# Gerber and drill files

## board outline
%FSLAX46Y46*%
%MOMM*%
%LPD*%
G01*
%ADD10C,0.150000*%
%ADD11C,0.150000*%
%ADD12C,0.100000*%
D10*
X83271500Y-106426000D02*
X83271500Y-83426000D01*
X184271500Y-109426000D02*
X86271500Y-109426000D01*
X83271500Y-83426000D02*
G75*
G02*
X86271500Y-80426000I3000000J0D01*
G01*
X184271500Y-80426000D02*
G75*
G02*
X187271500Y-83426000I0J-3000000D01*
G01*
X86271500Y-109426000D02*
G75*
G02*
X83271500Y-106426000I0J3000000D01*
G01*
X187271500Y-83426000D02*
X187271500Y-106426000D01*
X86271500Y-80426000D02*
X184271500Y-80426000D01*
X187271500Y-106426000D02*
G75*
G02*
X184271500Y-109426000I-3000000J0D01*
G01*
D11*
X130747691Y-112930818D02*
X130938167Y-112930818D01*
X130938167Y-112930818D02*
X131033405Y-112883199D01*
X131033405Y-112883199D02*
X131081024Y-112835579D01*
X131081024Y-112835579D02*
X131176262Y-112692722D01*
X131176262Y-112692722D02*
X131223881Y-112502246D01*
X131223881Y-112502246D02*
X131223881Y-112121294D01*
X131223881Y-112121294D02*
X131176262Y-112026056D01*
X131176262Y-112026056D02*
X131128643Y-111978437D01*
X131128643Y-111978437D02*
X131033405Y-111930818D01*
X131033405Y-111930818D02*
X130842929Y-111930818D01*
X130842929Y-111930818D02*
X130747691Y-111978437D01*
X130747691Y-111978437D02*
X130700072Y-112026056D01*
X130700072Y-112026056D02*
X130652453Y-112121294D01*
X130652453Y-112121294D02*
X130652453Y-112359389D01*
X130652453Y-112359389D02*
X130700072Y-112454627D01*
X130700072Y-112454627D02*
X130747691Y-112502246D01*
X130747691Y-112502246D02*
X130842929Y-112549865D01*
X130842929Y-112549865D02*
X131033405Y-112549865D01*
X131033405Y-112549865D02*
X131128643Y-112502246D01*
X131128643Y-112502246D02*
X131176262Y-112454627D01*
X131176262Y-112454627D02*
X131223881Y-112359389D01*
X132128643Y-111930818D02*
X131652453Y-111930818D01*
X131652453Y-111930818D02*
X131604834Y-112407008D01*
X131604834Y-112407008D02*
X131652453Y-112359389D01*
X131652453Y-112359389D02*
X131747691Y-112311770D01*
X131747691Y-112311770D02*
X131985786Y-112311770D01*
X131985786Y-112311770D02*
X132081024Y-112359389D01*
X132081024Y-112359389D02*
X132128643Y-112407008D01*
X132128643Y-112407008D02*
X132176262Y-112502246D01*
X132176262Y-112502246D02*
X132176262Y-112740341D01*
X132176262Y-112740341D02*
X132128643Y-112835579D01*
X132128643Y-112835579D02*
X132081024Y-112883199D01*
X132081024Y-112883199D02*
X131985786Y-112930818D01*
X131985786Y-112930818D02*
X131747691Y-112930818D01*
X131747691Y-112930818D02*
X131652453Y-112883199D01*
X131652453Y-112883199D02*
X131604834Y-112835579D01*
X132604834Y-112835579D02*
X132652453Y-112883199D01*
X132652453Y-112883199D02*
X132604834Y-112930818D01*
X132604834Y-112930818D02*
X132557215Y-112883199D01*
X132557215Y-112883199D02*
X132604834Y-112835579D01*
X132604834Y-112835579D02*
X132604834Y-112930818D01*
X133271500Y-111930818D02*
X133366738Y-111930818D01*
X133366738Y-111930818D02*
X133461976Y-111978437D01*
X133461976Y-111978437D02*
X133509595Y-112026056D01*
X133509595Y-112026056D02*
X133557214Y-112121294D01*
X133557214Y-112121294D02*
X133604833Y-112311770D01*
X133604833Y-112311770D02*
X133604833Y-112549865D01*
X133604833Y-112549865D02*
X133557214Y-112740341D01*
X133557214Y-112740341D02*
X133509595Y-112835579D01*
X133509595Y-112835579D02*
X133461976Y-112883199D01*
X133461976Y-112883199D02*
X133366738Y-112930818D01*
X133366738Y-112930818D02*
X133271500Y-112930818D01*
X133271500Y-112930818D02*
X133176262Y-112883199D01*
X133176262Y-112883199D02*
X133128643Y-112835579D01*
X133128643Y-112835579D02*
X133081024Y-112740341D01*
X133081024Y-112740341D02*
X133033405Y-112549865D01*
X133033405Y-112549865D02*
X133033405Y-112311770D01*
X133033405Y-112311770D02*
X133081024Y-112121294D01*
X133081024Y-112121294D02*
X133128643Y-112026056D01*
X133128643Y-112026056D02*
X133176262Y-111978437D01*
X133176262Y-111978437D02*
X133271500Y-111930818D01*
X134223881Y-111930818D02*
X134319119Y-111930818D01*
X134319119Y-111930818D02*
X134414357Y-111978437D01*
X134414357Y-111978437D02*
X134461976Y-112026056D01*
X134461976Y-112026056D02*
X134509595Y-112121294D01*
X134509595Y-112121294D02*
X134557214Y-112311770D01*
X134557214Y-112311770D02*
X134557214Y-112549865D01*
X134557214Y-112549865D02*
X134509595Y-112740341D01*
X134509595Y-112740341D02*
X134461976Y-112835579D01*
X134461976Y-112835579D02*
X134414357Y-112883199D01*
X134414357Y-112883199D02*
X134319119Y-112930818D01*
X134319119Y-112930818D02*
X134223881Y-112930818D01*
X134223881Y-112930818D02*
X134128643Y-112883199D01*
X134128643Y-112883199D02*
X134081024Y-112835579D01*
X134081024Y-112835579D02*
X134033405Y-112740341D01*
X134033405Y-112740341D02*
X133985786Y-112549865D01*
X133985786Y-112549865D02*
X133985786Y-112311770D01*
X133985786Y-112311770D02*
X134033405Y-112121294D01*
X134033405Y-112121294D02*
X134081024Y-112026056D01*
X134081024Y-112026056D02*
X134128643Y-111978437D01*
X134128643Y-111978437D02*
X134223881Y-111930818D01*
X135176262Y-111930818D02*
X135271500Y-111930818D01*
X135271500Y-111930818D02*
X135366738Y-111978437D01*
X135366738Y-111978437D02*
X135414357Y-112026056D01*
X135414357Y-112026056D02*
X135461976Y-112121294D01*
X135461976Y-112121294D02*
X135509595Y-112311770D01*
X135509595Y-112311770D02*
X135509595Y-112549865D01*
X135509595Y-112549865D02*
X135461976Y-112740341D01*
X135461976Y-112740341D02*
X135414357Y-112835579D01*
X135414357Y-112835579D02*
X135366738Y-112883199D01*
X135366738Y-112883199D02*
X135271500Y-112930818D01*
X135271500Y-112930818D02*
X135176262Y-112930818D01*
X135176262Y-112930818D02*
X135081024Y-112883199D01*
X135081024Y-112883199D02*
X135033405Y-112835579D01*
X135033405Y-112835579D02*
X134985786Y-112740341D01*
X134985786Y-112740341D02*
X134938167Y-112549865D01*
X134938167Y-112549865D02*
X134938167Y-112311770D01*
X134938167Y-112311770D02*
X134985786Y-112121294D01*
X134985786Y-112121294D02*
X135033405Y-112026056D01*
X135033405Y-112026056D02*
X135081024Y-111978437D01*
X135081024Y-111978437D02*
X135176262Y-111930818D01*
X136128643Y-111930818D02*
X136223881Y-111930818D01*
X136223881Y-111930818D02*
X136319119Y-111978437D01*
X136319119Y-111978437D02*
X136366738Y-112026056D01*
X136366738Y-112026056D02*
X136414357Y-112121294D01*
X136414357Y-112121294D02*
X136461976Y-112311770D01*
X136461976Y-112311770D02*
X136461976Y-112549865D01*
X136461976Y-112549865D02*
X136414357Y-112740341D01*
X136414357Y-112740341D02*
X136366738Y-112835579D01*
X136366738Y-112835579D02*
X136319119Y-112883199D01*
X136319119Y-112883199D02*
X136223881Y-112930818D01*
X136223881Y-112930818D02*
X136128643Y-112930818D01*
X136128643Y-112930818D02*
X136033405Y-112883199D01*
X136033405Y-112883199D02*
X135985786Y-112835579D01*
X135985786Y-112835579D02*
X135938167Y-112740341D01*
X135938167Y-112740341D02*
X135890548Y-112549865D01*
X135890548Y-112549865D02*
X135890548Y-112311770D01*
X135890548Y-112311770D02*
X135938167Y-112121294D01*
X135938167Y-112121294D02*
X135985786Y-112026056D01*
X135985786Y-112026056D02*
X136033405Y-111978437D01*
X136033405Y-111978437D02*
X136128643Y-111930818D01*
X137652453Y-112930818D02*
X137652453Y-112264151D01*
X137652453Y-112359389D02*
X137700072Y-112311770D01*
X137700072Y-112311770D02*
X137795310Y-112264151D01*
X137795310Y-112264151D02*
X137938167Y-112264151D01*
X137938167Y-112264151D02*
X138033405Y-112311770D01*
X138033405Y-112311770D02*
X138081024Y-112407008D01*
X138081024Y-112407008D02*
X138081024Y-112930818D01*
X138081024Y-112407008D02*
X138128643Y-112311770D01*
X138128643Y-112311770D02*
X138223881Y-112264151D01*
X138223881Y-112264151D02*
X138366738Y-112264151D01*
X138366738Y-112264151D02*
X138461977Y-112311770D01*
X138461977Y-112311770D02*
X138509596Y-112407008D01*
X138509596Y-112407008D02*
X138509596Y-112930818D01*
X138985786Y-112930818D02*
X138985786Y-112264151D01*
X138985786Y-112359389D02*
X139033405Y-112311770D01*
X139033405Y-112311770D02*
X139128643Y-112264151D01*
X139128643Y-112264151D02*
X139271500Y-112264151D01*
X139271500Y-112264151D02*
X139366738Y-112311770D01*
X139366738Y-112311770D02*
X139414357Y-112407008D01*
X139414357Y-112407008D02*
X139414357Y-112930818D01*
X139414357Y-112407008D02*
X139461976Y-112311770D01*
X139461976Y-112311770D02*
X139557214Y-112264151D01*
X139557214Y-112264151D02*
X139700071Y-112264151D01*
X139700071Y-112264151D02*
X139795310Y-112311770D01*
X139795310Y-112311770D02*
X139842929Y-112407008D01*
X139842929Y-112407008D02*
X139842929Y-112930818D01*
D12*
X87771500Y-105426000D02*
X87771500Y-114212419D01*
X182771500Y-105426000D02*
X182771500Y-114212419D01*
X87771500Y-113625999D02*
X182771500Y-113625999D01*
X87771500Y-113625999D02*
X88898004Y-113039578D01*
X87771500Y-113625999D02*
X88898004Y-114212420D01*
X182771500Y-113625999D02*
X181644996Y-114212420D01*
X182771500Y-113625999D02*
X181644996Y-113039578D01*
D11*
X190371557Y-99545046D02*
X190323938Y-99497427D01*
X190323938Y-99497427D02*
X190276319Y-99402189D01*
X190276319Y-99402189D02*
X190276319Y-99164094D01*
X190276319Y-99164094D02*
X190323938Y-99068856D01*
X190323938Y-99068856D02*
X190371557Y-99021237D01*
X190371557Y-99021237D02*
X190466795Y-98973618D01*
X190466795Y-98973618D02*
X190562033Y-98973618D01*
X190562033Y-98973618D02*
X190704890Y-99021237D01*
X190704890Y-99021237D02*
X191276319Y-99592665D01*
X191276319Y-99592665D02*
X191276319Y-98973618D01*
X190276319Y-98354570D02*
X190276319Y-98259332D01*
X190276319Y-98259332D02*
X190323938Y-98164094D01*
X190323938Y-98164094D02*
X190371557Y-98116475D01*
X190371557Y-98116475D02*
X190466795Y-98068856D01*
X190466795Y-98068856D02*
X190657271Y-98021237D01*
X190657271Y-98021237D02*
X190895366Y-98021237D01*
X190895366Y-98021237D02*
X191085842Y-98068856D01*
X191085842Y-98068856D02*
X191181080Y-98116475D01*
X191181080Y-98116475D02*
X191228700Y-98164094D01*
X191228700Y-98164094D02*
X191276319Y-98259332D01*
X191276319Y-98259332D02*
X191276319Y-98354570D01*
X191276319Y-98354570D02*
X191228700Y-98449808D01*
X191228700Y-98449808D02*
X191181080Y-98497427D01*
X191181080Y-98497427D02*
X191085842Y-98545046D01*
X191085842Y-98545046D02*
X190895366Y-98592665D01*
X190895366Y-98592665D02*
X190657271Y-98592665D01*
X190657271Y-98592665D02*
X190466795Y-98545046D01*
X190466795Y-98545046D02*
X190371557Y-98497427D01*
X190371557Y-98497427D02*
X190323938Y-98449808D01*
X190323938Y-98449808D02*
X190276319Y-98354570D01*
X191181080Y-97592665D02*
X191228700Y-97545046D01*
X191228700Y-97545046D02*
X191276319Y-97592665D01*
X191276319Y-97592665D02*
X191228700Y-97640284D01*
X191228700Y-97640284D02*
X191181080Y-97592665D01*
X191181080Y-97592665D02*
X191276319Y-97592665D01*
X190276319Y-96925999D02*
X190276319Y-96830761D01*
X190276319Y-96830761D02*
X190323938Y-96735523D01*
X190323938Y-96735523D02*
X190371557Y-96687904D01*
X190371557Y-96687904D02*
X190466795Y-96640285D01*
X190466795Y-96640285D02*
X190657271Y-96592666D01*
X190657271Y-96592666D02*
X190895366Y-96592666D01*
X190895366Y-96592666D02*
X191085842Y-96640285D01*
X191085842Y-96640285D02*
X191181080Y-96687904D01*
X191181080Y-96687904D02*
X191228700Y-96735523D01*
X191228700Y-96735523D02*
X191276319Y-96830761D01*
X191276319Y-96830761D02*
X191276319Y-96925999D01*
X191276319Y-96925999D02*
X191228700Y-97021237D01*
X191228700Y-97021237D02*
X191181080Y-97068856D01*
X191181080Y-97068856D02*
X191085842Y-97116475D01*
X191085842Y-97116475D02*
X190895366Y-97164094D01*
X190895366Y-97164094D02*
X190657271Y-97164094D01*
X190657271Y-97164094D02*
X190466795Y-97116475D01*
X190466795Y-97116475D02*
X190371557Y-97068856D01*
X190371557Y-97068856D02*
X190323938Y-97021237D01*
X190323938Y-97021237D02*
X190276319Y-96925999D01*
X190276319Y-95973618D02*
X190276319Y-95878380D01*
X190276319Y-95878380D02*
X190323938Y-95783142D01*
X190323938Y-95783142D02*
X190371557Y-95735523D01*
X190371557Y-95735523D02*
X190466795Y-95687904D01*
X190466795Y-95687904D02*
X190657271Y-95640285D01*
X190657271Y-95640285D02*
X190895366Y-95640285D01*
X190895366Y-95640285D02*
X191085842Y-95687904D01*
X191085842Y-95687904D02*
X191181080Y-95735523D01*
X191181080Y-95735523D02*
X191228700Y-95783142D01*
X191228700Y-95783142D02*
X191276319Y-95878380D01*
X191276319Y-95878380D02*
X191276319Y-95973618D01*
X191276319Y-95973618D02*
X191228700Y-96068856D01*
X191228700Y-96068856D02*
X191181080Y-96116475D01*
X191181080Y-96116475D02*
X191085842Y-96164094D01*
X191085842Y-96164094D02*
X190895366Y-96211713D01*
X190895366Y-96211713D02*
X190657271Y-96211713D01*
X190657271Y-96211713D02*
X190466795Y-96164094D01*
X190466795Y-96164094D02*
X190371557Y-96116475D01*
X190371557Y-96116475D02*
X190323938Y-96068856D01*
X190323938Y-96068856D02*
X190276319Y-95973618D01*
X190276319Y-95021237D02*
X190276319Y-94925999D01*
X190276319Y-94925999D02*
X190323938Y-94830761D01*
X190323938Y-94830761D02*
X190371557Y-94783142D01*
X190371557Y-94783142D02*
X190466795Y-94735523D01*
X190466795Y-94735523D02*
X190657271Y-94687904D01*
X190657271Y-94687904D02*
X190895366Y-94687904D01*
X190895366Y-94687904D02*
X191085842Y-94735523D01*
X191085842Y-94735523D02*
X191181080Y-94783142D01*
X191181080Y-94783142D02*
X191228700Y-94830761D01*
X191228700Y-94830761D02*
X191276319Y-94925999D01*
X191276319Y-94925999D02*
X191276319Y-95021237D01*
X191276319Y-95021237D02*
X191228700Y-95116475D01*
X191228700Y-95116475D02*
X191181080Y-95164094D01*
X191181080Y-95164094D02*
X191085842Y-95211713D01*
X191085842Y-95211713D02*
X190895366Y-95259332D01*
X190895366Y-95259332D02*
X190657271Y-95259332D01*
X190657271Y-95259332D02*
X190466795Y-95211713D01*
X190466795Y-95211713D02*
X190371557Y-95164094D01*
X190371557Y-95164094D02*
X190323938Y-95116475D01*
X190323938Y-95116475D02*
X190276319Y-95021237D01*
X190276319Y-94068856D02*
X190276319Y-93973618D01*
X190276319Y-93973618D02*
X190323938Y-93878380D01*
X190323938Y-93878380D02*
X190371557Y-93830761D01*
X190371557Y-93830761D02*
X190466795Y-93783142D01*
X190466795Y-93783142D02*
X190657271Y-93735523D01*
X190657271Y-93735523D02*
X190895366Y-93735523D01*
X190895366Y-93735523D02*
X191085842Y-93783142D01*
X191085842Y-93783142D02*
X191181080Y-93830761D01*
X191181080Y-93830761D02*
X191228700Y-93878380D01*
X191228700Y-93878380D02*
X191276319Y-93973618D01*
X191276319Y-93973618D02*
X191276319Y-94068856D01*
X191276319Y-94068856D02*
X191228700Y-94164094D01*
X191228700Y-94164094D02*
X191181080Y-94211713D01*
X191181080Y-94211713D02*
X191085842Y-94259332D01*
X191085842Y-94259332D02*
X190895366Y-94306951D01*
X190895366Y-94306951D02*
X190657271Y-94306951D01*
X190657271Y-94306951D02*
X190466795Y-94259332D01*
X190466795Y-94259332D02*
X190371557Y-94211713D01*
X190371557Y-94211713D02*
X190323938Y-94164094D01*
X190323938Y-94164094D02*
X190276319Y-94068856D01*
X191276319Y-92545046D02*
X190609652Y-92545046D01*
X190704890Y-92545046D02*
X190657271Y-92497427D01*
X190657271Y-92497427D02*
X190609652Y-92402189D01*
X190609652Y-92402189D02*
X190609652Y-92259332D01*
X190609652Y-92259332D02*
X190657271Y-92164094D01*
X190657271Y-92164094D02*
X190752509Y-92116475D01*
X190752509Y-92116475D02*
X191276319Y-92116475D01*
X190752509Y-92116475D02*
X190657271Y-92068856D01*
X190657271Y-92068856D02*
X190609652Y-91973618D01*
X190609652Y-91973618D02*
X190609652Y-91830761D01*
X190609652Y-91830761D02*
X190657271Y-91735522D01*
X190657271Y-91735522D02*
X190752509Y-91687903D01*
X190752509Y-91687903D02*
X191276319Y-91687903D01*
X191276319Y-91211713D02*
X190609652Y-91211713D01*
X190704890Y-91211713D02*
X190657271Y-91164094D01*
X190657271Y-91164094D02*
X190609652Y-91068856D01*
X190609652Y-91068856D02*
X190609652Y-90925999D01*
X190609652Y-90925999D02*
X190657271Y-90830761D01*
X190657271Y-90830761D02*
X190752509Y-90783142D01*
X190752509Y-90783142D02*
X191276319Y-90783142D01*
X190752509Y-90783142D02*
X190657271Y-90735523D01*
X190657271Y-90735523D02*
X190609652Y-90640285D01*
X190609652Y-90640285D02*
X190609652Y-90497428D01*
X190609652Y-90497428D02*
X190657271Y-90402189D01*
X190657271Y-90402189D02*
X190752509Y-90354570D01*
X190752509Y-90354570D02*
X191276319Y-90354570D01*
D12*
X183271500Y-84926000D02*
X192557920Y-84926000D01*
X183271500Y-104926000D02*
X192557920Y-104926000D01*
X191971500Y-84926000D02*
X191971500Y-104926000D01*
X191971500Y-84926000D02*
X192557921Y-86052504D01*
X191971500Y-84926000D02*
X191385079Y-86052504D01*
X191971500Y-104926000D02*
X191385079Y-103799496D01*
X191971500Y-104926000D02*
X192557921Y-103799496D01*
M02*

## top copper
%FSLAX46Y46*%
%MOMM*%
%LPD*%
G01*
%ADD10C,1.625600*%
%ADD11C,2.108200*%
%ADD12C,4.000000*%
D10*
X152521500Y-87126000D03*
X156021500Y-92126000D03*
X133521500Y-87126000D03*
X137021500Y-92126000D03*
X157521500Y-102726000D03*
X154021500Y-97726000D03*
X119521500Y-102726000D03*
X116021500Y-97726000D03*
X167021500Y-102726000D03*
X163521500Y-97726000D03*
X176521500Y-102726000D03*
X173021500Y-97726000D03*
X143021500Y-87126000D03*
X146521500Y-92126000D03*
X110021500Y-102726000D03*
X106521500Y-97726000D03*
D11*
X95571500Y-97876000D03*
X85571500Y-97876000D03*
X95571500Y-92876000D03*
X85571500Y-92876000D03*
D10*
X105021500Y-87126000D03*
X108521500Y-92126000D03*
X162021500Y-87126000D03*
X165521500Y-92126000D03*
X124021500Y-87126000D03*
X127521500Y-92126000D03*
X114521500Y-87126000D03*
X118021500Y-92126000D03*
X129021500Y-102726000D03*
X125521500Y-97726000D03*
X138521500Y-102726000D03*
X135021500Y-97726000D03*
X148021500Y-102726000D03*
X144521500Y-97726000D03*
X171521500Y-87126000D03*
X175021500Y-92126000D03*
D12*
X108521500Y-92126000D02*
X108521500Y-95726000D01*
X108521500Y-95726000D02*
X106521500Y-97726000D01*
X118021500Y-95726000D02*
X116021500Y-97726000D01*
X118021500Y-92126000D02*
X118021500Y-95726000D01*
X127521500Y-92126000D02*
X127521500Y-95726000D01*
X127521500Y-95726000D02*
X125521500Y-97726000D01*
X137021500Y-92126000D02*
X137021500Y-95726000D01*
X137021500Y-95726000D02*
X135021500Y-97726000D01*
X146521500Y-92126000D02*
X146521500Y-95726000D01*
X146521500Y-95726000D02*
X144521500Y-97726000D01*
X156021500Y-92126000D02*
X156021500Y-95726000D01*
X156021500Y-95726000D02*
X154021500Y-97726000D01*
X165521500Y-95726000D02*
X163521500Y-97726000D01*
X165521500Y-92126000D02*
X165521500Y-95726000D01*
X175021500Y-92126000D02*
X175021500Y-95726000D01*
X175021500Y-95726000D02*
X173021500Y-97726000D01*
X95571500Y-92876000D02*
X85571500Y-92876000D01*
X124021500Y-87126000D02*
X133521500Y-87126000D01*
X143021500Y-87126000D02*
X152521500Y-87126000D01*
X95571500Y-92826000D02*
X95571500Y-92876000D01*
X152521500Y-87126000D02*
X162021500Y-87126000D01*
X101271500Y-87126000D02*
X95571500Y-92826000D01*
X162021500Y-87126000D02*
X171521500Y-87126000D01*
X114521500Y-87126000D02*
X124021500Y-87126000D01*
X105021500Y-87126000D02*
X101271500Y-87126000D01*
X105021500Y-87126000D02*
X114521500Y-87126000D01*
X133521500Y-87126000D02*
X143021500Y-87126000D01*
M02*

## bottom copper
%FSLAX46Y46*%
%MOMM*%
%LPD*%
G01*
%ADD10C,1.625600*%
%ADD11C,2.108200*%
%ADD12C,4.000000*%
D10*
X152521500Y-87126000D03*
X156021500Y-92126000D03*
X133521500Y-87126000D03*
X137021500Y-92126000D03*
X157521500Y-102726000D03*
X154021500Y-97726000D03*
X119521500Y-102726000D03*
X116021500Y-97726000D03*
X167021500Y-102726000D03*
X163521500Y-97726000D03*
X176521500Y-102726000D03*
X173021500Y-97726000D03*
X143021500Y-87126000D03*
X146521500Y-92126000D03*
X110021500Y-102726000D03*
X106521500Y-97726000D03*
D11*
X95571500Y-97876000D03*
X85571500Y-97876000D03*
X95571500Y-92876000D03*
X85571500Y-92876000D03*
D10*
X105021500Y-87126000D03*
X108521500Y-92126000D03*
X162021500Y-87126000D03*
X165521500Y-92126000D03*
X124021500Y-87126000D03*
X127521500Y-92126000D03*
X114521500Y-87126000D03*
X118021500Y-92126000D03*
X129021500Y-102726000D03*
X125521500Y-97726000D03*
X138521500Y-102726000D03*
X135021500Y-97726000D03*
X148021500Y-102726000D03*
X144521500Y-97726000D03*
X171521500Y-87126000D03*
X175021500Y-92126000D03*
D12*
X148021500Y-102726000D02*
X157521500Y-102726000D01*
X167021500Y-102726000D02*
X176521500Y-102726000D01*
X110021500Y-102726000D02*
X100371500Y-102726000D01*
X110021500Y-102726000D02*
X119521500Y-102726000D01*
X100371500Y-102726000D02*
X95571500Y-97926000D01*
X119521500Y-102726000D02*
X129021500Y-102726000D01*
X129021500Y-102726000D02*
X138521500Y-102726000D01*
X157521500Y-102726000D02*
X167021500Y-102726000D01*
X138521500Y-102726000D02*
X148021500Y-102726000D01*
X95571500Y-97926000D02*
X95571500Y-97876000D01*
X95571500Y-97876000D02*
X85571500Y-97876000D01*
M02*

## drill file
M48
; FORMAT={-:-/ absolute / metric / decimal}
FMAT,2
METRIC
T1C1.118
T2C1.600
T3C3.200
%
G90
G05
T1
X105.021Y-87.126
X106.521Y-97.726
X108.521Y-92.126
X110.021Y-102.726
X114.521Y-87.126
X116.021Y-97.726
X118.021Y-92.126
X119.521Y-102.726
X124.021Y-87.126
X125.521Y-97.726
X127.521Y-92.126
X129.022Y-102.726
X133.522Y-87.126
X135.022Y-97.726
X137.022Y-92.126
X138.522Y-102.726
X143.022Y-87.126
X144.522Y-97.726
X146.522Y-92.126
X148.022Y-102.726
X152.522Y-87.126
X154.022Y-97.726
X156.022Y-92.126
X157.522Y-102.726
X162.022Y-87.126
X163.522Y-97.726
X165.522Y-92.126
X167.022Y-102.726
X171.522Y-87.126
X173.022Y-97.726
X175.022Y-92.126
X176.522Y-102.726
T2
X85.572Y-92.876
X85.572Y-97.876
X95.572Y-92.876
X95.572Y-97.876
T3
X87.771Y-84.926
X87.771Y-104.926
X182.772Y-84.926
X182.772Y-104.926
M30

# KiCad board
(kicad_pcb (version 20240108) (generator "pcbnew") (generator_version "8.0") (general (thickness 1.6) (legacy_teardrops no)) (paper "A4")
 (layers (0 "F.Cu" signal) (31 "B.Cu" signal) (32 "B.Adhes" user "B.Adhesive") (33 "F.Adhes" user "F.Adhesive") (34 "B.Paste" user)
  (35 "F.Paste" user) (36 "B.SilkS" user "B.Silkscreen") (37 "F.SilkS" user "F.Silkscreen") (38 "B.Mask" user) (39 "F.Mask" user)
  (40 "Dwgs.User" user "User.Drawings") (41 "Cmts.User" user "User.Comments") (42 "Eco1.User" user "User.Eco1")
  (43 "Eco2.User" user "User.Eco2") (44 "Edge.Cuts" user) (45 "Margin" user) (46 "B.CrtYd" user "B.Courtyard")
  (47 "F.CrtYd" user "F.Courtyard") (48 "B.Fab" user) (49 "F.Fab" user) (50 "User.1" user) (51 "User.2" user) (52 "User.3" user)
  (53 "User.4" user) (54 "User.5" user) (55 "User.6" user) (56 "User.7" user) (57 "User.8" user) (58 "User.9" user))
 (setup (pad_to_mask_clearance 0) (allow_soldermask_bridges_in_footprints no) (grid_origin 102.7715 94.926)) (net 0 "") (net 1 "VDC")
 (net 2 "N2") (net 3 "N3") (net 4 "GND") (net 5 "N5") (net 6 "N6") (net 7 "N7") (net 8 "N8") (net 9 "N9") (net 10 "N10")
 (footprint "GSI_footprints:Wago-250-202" (layer "F.Cu") (at 152.5215 87.126 180)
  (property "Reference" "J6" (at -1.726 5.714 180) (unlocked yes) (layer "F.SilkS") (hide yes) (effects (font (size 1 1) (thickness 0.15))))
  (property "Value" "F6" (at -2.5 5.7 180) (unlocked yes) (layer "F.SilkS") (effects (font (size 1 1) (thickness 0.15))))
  (pad "1" thru_hole circle (at 0 0 180) (size 1.6256 1.6256) (drill 1.1176) (layers "*.Cu" "*.Mask") (remove_unused_layers no)
   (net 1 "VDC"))
  (pad "2" thru_hole circle (at -3.5 -5 180) (size 1.6256 1.6256) (drill 1.1176) (layers "*.Cu" "*.Mask") (remove_unused_layers no)
   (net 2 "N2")))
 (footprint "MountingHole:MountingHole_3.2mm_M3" (layer "F.Cu") (at 182.7715 104.926)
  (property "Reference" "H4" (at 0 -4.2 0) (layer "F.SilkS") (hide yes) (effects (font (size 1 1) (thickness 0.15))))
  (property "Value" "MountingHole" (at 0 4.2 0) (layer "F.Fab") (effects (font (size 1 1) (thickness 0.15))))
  (pad "" np_thru_hole circle (at 0 0) (size 3.2 3.2) (drill 3.2) (layers "*.Cu" "*.Mask")))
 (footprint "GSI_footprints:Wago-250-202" (layer "F.Cu") (at 133.5215 87.126 180)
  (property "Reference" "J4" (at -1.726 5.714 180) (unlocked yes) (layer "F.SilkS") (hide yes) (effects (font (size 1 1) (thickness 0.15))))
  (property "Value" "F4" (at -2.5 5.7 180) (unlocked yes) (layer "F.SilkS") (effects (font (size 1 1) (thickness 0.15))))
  (pad "1" thru_hole circle (at 0 0 180) (size 1.6256 1.6256) (drill 1.1176) (layers "*.Cu" "*.Mask") (remove_unused_layers no)
   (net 1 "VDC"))
  (pad "2" thru_hole circle (at -3.5 -5 180) (size 1.6256 1.6256) (drill 1.1176) (layers "*.Cu" "*.Mask") (remove_unused_layers no)
   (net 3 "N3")))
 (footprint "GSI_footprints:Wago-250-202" (layer "F.Cu") (at 157.5215 102.726)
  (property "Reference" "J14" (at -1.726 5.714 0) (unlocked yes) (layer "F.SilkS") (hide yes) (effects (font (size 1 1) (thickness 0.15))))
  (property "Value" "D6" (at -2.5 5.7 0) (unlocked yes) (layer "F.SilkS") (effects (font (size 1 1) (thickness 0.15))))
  (pad "1" thru_hole circle (at 0 0) (size 1.6256 1.6256) (drill 1.1176) (layers "*.Cu" "*.Mask") (remove_unused_layers no) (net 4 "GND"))
  (pad "2" thru_hole circle (at -3.5 -5) (size 1.6256 1.6256) (drill 1.1176) (layers "*.Cu" "*.Mask") (remove_unused_layers no) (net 2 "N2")))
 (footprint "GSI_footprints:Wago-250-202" (layer "F.Cu") (at 119.5215 102.726)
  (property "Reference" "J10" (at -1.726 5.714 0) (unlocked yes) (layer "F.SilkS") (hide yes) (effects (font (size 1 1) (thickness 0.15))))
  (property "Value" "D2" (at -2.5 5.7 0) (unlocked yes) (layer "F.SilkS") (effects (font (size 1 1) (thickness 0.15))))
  (pad "1" thru_hole circle (at 0 0) (size 1.6256 1.6256) (drill 1.1176) (layers "*.Cu" "*.Mask") (remove_unused_layers no) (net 4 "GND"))
  (pad "2" thru_hole circle (at -3.5 -5) (size 1.6256 1.6256) (drill 1.1176) (layers "*.Cu" "*.Mask") (remove_unused_layers no) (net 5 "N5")))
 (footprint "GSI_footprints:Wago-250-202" (layer "F.Cu") (at 167.0215 102.726)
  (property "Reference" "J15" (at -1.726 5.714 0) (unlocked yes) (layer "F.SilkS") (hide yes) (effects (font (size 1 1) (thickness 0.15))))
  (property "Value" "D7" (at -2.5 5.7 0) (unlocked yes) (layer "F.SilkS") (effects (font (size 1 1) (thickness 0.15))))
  (pad "1" thru_hole circle (at 0 0) (size 1.6256 1.6256) (drill 1.1176) (layers "*.Cu" "*.Mask") (remove_unused_layers no) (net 4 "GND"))
  (pad "2" thru_hole circle (at -3.5 -5) (size 1.6256 1.6256) (drill 1.1176) (layers "*.Cu" "*.Mask") (remove_unused_layers no) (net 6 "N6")))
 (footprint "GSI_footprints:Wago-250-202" (layer "F.Cu") (at 176.5215 102.726)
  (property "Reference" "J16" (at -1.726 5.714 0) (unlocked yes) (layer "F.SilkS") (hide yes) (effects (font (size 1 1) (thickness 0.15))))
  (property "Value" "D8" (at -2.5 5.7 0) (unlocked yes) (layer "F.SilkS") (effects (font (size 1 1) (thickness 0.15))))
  (pad "1" thru_hole circle (at 0 0) (size 1.6256 1.6256) (drill 1.1176) (layers "*.Cu" "*.Mask") (remove_unused_layers no) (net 4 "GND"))
  (pad "2" thru_hole circle (at -3.5 -5) (size 1.6256 1.6256) (drill 1.1176) (layers "*.Cu" "*.Mask") (remove_unused_layers no) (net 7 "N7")))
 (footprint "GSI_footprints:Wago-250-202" (layer "F.Cu") (at 143.0215 87.126 180)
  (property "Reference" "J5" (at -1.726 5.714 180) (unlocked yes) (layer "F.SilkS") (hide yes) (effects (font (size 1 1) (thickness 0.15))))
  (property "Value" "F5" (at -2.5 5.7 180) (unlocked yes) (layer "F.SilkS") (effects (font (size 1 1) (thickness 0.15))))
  (pad "1" thru_hole circle (at 0 0 180) (size 1.6256 1.6256) (drill 1.1176) (layers "*.Cu" "*.Mask") (remove_unused_layers no)
   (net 1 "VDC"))
  (pad "2" thru_hole circle (at -3.5 -5 180) (size 1.6256 1.6256) (drill 1.1176) (layers "*.Cu" "*.Mask") (remove_unused_layers no)
   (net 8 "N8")))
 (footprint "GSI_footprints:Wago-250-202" (layer "F.Cu") (at 110.0215 102.726)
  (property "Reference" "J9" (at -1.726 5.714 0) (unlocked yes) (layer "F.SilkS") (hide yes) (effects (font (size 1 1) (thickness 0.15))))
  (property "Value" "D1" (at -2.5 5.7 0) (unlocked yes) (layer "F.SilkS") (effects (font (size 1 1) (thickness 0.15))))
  (pad "1" thru_hole circle (at 0 0) (size 1.6256 1.6256) (drill 1.1176) (layers "*.Cu" "*.Mask") (remove_unused_layers no) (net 4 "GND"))
  (pad "2" thru_hole circle (at -3.5 -5) (size 1.6256 1.6256) (drill 1.1176) (layers "*.Cu" "*.Mask") (remove_unused_layers no) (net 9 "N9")))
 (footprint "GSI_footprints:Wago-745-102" (layer "F.Cu") (at 85.5715 97.876 -90)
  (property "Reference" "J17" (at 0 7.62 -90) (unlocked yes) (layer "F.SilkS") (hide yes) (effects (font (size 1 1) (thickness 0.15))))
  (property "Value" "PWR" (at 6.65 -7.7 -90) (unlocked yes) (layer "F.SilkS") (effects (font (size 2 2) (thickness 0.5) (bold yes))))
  (pad "1" thru_hole circle (at 0 -10 270) (size 2.1082 2.1082) (drill 1.6002) (layers "*.Cu" "*.Mask") (remove_unused_layers no)
   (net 4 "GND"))
  (pad "1" thru_hole circle (at 0 0 270) (size 2.1082 2.1082) (drill 1.6002) (layers "*.Cu" "*.Mask") (remove_unused_layers no)
   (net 4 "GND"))
  (pad "2" thru_hole circle (at -5 -10 270) (size 2.1082 2.1082) (drill 1.6002) (layers "*.Cu" "*.Mask") (remove_unused_layers no)
   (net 1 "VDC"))
  (pad "2" thru_hole circle (at -5 0 270) (size 2.1082 2.1082) (drill 1.6002) (layers "*.Cu" "*.Mask") (remove_unused_layers no)
   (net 1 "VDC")))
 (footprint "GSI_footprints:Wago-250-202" (layer "F.Cu") (at 105.0215 87.126 180)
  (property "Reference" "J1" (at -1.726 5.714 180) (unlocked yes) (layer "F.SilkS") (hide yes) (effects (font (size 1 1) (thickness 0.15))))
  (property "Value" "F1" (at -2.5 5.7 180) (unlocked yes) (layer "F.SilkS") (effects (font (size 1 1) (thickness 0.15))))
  (pad "1" thru_hole circle (at 0 0 180) (size 1.6256 1.6256) (drill 1.1176) (layers "*.Cu" "*.Mask") (remove_unused_layers no)
   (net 1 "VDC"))
  (pad "2" thru_hole circle (at -3.5 -5 180) (size 1.6256 1.6256) (drill 1.1176) (layers "*.Cu" "*.Mask") (remove_unused_layers no)
   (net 9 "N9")))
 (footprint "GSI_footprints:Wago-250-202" (layer "F.Cu") (at 162.0215 87.126 180)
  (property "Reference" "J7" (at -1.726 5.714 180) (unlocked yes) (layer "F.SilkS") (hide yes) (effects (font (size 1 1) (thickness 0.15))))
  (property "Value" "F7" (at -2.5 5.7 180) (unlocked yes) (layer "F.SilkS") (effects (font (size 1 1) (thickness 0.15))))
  (pad "1" thru_hole circle (at 0 0 180) (size 1.6256 1.6256) (drill 1.1176) (layers "*.Cu" "*.Mask") (remove_unused_layers no)
   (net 1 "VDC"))
  (pad "2" thru_hole circle (at -3.5 -5 180) (size 1.6256 1.6256) (drill 1.1176) (layers "*.Cu" "*.Mask") (remove_unused_layers no)
   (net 6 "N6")))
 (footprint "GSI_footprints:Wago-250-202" (layer "F.Cu") (at 124.0215 87.126 180)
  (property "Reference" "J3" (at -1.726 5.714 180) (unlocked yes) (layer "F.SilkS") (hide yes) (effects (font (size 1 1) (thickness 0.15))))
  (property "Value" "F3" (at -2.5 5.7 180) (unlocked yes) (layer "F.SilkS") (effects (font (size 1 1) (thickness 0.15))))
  (pad "1" thru_hole circle (at 0 0 180) (size 1.6256 1.6256) (drill 1.1176) (layers "*.Cu" "*.Mask") (remove_unused_layers no)
   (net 1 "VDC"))
  (pad "2" thru_hole circle (at -3.5 -5 180) (size 1.6256 1.6256) (drill 1.1176) (layers "*.Cu" "*.Mask") (remove_unused_layers no)
   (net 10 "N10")))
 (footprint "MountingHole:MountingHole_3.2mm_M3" (layer "F.Cu") (at 182.7715 84.926)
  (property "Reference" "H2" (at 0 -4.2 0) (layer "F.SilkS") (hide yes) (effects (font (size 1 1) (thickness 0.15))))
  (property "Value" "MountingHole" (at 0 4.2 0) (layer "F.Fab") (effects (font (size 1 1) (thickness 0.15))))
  (pad "" np_thru_hole circle (at 0 0) (size 3.2 3.2) (drill 3.2) (layers "*.Cu" "*.Mask")))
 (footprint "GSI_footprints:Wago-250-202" (layer "F.Cu") (at 114.5215 87.126 180)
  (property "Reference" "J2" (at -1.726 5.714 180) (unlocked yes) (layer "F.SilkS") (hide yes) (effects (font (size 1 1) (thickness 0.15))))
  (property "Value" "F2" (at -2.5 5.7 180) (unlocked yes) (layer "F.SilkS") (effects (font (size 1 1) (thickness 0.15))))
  (pad "1" thru_hole circle (at 0 0 180) (size 1.6256 1.6256) (drill 1.1176) (layers "*.Cu" "*.Mask") (remove_unused_layers no)
   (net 1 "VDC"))
  (pad "2" thru_hole circle (at -3.5 -5 180) (size 1.6256 1.6256) (drill 1.1176) (layers "*.Cu" "*.Mask") (remove_unused_layers no)
   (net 5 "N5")))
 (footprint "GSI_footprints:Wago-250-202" (layer "F.Cu") (at 129.0215 102.726)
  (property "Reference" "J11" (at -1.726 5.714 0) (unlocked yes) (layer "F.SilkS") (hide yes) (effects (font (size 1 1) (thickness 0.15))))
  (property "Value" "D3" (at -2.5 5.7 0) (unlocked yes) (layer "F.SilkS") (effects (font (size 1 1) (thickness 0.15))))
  (pad "1" thru_hole circle (at 0 0) (size 1.6256 1.6256) (drill 1.1176) (layers "*.Cu" "*.Mask") (remove_unused_layers no) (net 4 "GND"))
  (pad "2" thru_hole circle (at -3.5 -5) (size 1.6256 1.6256) (drill 1.1176) (layers "*.Cu" "*.Mask") (remove_unused_layers no)
   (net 10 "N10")))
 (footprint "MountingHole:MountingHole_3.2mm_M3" (layer "F.Cu") (at 87.7715 104.926)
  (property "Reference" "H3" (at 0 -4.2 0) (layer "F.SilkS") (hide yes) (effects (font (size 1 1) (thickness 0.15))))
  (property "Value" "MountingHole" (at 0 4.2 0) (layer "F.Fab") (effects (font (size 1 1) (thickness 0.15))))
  (pad "" np_thru_hole circle (at 0 0) (size 3.2 3.2) (drill 3.2) (layers "*.Cu" "*.Mask")))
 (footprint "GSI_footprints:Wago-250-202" (layer "F.Cu") (at 138.5215 102.726)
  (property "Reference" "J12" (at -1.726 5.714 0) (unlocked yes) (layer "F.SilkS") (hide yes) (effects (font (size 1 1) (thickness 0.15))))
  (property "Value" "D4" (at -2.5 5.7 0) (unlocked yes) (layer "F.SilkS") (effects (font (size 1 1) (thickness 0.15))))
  (pad "1" thru_hole circle (at 0 0) (size 1.6256 1.6256) (drill 1.1176) (layers "*.Cu" "*.Mask") (remove_unused_layers no) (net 4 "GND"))
  (pad "2" thru_hole circle (at -3.5 -5) (size 1.6256 1.6256) (drill 1.1176) (layers "*.Cu" "*.Mask") (remove_unused_layers no) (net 3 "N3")))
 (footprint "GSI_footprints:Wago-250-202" (layer "F.Cu") (at 148.0215 102.726)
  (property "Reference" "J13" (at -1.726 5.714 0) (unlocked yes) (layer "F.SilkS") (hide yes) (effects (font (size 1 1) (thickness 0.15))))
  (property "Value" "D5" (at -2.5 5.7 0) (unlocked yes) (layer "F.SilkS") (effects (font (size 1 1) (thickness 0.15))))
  (pad "1" thru_hole circle (at 0 0) (size 1.6256 1.6256) (drill 1.1176) (layers "*.Cu" "*.Mask") (remove_unused_layers no) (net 4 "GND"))
  (pad "2" thru_hole circle (at -3.5 -5) (size 1.6256 1.6256) (drill 1.1176) (layers "*.Cu" "*.Mask") (remove_unused_layers no) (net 8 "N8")))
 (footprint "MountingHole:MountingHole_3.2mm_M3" (layer "F.Cu") (at 87.7715 84.926)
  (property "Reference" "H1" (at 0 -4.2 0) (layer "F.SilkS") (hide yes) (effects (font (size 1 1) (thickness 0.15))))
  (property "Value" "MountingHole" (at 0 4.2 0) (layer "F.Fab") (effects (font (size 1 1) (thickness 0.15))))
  (pad "" np_thru_hole circle (at 0 0) (size 3.2 3.2) (drill 3.2) (layers "*.Cu" "*.Mask")))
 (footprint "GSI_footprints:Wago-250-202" (layer "F.Cu") (at 171.5215 87.126 180)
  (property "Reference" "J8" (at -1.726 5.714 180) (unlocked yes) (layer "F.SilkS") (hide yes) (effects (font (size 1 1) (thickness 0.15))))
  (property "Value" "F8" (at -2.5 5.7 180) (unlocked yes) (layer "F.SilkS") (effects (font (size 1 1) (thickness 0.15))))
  (pad "1" thru_hole circle (at 0 0 180) (size 1.6256 1.6256) (drill 1.1176) (layers "*.Cu" "*.Mask") (remove_unused_layers no)
   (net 1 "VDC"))
  (pad "2" thru_hole circle (at -3.5 -5 180) (size 1.6256 1.6256) (drill 1.1176) (layers "*.Cu" "*.Mask") (remove_unused_layers no)
   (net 7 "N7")))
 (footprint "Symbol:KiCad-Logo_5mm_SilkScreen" (layer "B.Cu") (at 98.3715 105.126 180)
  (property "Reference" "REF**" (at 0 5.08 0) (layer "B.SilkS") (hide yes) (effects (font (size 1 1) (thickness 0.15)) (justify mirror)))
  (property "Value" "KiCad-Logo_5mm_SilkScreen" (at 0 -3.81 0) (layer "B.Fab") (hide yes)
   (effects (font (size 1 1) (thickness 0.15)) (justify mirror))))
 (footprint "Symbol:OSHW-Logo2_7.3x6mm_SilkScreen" (layer "B.Cu") (at 172.0715 104.926 180)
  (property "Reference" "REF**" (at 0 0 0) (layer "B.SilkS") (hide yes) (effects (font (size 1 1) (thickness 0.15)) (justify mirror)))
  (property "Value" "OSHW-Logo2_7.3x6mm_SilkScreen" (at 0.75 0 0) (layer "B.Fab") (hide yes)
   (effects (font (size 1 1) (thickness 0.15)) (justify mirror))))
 (gr_line (start 83.2715 106.426) (end 83.2715 83.426) (stroke (width 0.15) (type default)) (layer "Edge.Cuts"))
 (gr_line (start 184.2715 109.426) (end 86.2715 109.426) (stroke (width 0.15) (type default)) (layer "Edge.Cuts"))
 (gr_arc (start 83.2715 83.426) (mid 84.15018 81.30468) (end 86.2715 80.426) (stroke (width 0.15) (type default)) (layer "Edge.Cuts"))
 (gr_arc (start 184.2715 80.426) (mid 186.39282 81.30468) (end 187.2715 83.426) (stroke (width 0.15) (type default)) (layer "Edge.Cuts"))
 (gr_arc (start 86.2715 109.426) (mid 84.15018 108.54732) (end 83.2715 106.426) (stroke (width 0.15) (type default)) (layer "Edge.Cuts"))
 (gr_line (start 187.2715 83.426) (end 187.2715 106.426) (stroke (width 0.15) (type default)) (layer "Edge.Cuts"))
 (gr_line (start 86.2715 80.426) (end 184.2715 80.426) (stroke (width 0.15) (type default)) (layer "Edge.Cuts"))
 (gr_arc (start 187.2715 106.426) (mid 186.39282 108.54732) (end 184.2715 109.426) (stroke (width 0.15) (type default)) (layer "Edge.Cuts"))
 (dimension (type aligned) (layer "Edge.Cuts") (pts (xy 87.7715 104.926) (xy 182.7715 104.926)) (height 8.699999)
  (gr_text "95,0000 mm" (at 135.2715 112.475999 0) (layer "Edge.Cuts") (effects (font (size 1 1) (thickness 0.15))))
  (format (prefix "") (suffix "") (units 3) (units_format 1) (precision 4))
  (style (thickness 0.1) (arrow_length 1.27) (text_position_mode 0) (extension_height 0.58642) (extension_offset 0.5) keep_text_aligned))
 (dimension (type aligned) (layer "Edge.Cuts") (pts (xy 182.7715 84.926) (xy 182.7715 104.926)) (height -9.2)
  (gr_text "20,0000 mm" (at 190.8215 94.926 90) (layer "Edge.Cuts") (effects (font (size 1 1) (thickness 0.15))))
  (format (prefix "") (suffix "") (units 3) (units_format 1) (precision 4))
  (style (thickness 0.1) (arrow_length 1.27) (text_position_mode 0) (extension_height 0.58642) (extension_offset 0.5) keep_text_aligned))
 (segment (start 108.5215 92.126) (end 108.5215 95.726) (width 4) (layer "F.Cu") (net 9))
 (segment (start 108.5215 95.726) (end 106.5215 97.726) (width 4) (layer "F.Cu") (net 9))
 (segment (start 118.0215 95.726) (end 116.0215 97.726) (width 4) (layer "F.Cu") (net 5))
 (segment (start 118.0215 92.126) (end 118.0215 95.726) (width 4) (layer "F.Cu") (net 5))
 (segment (start 127.5215 92.126) (end 127.5215 95.726) (width 4) (layer "F.Cu") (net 10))
 (segment (start 127.5215 95.726) (end 125.5215 97.726) (width 4) (layer "F.Cu") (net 10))
 (segment (start 137.0215 92.126) (end 137.0215 95.726) (width 4) (layer "F.Cu") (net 3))
 (segment (start 137.0215 95.726) (end 135.0215 97.726) (width 4) (layer "F.Cu") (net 3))
 (segment (start 146.5215 92.126) (end 146.5215 95.726) (width 4) (layer "F.Cu") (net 8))
 (segment (start 146.5215 95.726) (end 144.5215 97.726) (width 4) (layer "F.Cu") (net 8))
 (segment (start 156.0215 92.126) (end 156.0215 95.726) (width 4) (layer "F.Cu") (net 2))
 (segment (start 156.0215 95.726) (end 154.0215 97.726) (width 4) (layer "F.Cu") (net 2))
 (segment (start 165.5215 95.726) (end 163.5215 97.726) (width 4) (layer "F.Cu") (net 6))
 (segment (start 165.5215 92.126) (end 165.5215 95.726) (width 4) (layer "F.Cu") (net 6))
 (segment (start 175.0215 92.126) (end 175.0215 95.726) (width 4) (layer "F.Cu") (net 7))
 (segment (start 175.0215 95.726) (end 173.0215 97.726) (width 4) (layer "F.Cu") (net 7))
 (segment (start 95.5715 92.876) (end 85.5715 92.876) (width 4) (layer "F.Cu") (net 1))
 (segment (start 124.0215 87.126) (end 133.5215 87.126) (width 4) (layer "F.Cu") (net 1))
 (segment (start 143.0215 87.126) (end 152.5215 87.126) (width 4) (layer "F.Cu") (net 1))
 (segment (start 95.5715 92.826) (end 95.5715 92.876) (width 4) (layer "F.Cu") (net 1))
 (segment (start 152.5215 87.126) (end 162.0215 87.126) (width 4) (layer "F.Cu") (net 1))
 (segment (start 101.2715 87.126) (end 95.5715 92.826) (width 4) (layer "F.Cu") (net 1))
 (segment (start 162.0215 87.126) (end 171.5215 87.126) (width 4) (layer "F.Cu") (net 1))
 (segment (start 114.5215 87.126) (end 124.0215 87.126) (width 4) (layer "F.Cu") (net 1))
 (segment (start 105.0215 87.126) (end 101.2715 87.126) (width 4) (layer "F.Cu") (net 1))
 (segment (start 105.0215 87.126) (end 114.5215 87.126) (width 4) (layer "F.Cu") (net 1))
 (segment (start 133.5215 87.126) (end 143.0215 87.126) (width 4) (layer "F.Cu") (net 1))
 (segment (start 148.0215 102.726) (end 157.5215 102.726) (width 4) (layer "B.Cu") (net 4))
 (segment (start 167.0215 102.726) (end 176.5215 102.726) (width 4) (layer "B.Cu") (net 4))
 (segment (start 110.0215 102.726) (end 100.3715 102.726) (width 4) (layer "B.Cu") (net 4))
 (segment (start 110.0215 102.726) (end 119.5215 102.726) (width 4) (layer "B.Cu") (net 4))
 (segment (start 100.3715 102.726) (end 95.5715 97.926) (width 4) (layer "B.Cu") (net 4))
 (segment (start 119.5215 102.726) (end 129.0215 102.726) (width 4) (layer "B.Cu") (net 4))
 (segment (start 129.0215 102.726) (end 138.5215 102.726) (width 4) (layer "B.Cu") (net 4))
 (segment (start 157.5215 102.726) (end 167.0215 102.726) (width 4) (layer "B.Cu") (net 4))
 (segment (start 138.5215 102.726) (end 148.0215 102.726) (width 4) (layer "B.Cu") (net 4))
 (segment (start 95.5715 97.926) (end 95.5715 97.876) (width 4) (layer "B.Cu") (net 4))
 (segment (start 95.5715 97.876) (end 85.5715 97.876) (width 4) (layer "B.Cu") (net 4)))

